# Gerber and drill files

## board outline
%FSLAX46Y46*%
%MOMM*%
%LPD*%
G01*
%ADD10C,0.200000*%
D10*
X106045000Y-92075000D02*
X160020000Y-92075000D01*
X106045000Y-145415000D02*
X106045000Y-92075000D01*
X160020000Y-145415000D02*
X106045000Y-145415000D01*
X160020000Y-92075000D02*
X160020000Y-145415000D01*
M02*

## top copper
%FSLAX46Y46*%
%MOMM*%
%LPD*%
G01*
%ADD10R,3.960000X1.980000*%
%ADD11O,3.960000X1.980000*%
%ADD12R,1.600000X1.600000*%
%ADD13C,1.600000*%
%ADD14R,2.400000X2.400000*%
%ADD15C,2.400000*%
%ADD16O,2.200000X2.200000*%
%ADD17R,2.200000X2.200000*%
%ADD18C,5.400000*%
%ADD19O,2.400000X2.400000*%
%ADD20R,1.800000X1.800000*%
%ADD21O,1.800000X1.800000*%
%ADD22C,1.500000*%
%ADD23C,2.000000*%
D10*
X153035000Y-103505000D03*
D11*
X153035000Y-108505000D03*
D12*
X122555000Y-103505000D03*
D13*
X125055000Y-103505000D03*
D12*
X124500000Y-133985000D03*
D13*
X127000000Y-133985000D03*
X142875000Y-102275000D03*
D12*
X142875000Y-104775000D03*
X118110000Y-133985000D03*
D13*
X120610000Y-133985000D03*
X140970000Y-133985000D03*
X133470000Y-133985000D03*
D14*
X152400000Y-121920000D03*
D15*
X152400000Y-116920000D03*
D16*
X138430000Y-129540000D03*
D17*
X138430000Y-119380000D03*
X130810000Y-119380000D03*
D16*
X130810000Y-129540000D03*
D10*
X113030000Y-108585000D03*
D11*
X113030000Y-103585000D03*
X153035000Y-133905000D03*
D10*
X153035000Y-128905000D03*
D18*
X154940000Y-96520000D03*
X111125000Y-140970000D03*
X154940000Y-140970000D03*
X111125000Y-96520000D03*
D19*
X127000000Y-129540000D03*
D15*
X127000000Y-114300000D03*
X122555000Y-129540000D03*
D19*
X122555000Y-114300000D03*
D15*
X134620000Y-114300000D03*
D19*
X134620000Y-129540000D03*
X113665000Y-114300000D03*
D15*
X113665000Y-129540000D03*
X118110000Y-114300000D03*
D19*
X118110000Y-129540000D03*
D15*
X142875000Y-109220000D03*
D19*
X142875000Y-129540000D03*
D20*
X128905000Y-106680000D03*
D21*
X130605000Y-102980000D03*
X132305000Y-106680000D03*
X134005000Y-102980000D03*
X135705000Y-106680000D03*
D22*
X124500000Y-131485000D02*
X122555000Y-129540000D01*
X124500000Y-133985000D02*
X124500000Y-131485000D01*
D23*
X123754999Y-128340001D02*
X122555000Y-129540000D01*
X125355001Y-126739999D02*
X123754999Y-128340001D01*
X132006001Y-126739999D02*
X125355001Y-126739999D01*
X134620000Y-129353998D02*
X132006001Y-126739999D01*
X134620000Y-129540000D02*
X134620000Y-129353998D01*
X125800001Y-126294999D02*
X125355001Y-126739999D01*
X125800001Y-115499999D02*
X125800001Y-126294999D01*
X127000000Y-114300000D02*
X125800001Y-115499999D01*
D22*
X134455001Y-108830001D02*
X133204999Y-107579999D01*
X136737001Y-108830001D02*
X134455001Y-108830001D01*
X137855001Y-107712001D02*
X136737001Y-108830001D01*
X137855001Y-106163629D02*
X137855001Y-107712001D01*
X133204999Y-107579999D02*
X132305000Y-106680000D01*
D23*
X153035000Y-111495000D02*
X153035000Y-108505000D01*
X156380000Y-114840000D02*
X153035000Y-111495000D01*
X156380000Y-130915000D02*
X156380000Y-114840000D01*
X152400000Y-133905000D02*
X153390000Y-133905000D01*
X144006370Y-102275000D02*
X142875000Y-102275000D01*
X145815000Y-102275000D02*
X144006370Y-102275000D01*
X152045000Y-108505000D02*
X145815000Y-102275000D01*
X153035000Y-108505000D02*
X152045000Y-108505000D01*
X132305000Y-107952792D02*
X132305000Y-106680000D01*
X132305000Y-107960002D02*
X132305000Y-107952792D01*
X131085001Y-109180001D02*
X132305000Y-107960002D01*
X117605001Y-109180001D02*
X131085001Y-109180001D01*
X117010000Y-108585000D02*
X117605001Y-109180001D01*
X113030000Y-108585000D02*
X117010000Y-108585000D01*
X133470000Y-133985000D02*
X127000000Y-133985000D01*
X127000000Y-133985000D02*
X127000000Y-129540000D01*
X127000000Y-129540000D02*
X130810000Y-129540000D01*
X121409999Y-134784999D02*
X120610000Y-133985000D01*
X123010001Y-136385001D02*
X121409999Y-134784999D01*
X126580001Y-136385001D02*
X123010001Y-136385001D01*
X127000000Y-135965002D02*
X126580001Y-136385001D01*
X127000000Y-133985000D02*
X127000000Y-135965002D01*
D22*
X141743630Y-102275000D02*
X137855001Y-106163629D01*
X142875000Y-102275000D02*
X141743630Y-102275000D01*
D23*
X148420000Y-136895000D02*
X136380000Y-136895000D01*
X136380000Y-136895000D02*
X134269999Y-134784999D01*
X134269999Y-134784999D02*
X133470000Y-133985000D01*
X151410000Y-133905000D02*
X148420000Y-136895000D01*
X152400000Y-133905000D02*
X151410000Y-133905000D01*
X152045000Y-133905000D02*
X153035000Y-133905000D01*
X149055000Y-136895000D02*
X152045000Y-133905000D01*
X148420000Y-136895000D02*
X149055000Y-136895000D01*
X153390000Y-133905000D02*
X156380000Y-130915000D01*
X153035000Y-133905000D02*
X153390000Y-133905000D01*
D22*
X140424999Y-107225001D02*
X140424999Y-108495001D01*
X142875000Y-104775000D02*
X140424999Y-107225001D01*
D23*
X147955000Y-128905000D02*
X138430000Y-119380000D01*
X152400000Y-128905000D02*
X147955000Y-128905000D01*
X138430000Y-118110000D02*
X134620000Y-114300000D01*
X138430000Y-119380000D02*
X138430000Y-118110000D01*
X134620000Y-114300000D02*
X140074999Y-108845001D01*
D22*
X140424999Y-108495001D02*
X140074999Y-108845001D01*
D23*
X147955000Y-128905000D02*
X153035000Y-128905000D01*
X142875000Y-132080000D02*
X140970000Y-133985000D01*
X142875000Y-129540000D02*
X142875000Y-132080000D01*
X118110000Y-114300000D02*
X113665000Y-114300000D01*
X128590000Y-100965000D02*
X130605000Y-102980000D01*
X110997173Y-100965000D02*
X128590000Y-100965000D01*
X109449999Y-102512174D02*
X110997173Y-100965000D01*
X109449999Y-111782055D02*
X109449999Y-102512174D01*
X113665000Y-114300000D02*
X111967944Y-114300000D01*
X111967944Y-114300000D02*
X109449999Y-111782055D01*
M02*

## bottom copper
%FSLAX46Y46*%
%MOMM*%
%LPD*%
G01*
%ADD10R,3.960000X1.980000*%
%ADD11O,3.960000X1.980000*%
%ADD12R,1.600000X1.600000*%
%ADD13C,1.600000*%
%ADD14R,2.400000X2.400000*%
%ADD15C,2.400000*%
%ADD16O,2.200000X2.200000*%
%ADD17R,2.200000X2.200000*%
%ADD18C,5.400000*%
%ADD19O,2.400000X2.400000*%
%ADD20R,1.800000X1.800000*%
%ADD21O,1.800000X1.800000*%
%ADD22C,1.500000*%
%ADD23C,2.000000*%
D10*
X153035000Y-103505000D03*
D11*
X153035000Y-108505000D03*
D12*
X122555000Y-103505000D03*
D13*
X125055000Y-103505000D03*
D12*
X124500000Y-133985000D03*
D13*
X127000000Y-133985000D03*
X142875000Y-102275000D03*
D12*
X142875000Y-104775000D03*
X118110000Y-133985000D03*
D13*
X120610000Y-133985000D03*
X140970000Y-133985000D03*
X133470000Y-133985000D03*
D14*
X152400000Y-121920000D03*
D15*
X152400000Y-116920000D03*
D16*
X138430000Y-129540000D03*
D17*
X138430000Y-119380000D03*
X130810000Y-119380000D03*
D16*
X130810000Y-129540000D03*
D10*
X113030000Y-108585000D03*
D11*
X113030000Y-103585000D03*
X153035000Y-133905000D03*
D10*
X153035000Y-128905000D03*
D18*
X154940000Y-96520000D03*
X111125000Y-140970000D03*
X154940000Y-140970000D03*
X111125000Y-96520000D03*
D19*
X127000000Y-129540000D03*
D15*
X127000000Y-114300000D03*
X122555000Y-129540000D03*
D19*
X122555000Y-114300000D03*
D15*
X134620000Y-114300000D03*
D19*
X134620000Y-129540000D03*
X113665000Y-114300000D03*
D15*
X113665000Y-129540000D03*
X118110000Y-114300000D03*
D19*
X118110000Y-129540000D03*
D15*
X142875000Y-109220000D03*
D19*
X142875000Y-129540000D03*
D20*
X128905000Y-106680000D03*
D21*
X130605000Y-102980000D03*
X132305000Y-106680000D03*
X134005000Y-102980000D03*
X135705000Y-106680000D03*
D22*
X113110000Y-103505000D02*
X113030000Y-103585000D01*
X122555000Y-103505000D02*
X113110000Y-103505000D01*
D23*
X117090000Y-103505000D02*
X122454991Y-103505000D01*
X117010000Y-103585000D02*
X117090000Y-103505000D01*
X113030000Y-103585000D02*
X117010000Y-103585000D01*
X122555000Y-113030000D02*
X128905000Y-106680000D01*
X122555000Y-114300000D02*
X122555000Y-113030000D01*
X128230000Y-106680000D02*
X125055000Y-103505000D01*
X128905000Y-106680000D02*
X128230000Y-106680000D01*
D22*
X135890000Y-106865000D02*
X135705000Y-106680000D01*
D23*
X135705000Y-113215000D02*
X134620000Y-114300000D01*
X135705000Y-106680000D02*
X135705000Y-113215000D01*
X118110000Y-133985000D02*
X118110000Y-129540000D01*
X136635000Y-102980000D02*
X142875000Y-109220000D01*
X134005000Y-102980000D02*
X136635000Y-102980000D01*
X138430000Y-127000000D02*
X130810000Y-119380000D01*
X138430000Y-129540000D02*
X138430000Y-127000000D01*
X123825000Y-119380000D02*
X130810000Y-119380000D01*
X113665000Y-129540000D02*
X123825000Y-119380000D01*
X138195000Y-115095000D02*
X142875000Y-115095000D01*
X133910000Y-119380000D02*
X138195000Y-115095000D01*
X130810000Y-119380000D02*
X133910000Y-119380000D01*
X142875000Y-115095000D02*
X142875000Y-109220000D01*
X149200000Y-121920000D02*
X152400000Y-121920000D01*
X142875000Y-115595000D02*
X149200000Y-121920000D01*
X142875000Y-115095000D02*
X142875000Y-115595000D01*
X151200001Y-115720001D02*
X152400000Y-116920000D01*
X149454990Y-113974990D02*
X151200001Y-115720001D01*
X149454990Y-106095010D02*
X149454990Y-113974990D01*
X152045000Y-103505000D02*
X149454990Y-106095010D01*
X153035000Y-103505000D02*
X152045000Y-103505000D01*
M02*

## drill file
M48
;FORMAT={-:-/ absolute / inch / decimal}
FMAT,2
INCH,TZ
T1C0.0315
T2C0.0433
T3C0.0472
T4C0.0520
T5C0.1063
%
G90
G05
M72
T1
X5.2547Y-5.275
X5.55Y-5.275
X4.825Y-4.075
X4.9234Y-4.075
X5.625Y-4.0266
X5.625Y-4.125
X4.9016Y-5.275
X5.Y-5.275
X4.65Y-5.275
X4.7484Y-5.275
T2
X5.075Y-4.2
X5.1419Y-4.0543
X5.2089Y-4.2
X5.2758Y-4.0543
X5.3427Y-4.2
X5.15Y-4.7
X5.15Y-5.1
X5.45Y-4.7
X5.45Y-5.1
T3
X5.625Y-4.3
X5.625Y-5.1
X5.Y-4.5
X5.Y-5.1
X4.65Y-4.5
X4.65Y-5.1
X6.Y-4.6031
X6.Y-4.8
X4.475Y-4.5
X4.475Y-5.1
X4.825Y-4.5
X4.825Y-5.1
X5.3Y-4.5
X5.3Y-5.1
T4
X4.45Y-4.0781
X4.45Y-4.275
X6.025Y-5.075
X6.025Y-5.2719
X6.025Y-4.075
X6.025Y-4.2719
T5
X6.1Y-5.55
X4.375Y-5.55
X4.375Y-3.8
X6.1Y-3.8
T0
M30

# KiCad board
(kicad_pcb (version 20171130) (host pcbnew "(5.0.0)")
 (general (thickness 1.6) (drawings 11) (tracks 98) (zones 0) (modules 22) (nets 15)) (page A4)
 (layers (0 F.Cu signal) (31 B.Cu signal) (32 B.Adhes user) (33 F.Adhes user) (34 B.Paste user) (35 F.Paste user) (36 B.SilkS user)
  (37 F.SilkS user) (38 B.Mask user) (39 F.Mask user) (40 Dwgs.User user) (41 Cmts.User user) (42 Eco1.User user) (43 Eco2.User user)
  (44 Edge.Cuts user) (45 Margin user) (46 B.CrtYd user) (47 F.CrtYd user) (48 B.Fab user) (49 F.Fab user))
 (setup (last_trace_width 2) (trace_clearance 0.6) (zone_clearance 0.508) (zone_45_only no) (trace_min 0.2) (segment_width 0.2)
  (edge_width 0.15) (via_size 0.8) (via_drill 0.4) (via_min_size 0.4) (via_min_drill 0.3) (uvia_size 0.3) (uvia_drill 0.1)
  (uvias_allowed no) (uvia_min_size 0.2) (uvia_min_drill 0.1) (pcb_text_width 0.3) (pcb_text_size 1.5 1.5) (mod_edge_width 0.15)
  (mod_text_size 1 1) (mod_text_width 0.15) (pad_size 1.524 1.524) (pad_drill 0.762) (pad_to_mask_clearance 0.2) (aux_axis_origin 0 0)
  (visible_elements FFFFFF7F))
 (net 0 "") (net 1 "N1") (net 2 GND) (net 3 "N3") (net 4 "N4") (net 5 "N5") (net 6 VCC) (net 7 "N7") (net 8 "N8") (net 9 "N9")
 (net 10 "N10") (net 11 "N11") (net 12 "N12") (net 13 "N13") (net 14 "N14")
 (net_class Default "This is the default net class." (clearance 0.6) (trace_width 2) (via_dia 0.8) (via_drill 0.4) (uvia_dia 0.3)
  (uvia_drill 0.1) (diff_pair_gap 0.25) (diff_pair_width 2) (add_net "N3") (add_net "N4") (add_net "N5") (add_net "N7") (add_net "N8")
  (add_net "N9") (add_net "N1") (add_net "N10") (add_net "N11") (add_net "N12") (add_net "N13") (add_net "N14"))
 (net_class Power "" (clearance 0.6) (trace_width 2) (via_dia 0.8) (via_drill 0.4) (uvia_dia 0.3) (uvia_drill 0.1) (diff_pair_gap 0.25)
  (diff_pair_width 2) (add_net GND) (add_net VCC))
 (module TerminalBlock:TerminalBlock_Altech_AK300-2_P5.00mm (layer F.Cu) (at 153.035 103.505 270)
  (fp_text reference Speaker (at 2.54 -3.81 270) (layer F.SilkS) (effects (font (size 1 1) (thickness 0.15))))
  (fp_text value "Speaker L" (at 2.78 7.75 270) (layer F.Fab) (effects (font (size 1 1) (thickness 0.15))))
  (pad 1 thru_hole rect (at 0 0 270) (size 1.98 3.96) (drill 1.32) (layers *.Cu *.Mask) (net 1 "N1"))
  (pad 2 thru_hole oval (at 5 0 270) (size 1.98 3.96) (drill 1.32) (layers *.Cu *.Mask) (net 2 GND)))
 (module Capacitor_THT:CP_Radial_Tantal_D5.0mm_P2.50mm (layer F.Cu) (at 122.555 103.505)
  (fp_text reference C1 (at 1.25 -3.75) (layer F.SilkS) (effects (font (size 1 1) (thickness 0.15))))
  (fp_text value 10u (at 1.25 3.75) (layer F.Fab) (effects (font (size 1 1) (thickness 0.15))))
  (pad 1 thru_hole rect (at 0 0) (size 1.6 1.6) (drill 0.8) (layers *.Cu *.Mask) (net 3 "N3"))
  (pad 2 thru_hole circle (at 2.5 0) (size 1.6 1.6) (drill 0.8) (layers *.Cu *.Mask) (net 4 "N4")))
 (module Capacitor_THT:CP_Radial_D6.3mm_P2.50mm (layer F.Cu) (at 124.5 133.985)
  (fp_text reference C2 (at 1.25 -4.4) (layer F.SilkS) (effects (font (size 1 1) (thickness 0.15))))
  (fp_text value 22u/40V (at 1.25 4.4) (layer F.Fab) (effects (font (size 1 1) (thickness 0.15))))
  (pad 1 thru_hole rect (at 0 0) (size 1.6 1.6) (drill 0.8) (layers *.Cu *.Mask) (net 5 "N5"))
  (pad 2 thru_hole circle (at 2.5 0) (size 1.6 1.6) (drill 0.8) (layers *.Cu *.Mask) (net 2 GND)))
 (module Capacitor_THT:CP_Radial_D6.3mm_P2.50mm (layer F.Cu) (at 142.875 104.775 90)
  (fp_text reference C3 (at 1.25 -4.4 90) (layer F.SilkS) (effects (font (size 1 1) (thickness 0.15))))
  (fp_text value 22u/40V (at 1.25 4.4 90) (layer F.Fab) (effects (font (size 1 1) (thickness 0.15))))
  (pad 2 thru_hole circle (at 2.5 0 90) (size 1.6 1.6) (drill 0.8) (layers *.Cu *.Mask) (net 2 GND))
  (pad 1 thru_hole rect (at 0 0 90) (size 1.6 1.6) (drill 0.8) (layers *.Cu *.Mask) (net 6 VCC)))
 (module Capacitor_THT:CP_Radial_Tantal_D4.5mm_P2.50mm (layer F.Cu) (at 118.11 133.985)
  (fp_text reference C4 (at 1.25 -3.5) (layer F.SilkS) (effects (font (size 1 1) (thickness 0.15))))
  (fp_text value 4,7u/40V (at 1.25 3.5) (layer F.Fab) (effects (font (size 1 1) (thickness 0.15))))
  (pad 1 thru_hole rect (at 0 0) (size 1.6 1.6) (drill 0.8) (layers *.Cu *.Mask) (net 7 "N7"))
  (pad 2 thru_hole circle (at 2.5 0) (size 1.6 1.6) (drill 0.8) (layers *.Cu *.Mask) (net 2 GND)))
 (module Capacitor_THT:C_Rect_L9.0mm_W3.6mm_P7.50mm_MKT (layer F.Cu) (at 140.97 133.985 180)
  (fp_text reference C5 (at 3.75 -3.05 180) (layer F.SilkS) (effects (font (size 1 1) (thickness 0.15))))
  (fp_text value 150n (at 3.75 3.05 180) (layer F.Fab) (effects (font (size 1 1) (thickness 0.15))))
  (pad 1 thru_hole circle (at 0 0 180) (size 1.6 1.6) (drill 0.8) (layers *.Cu *.Mask) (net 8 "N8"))
  (pad 2 thru_hole circle (at 7.5 0 180) (size 1.6 1.6) (drill 0.8) (layers *.Cu *.Mask) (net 2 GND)))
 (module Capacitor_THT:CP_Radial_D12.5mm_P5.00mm (layer F.Cu) (at 152.4 121.92 90)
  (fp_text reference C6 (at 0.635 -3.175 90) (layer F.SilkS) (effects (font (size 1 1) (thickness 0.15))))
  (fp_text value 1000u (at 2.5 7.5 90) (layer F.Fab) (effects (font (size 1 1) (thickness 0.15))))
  (pad 1 thru_hole rect (at 0 0 90) (size 2.4 2.4) (drill 1.2) (layers *.Cu *.Mask) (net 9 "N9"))
  (pad 2 thru_hole circle (at 5 0 90) (size 2.4 2.4) (drill 1.2) (layers *.Cu *.Mask) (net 1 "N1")))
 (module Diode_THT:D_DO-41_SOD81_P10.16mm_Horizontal (layer F.Cu) (at 138.43 119.38 270)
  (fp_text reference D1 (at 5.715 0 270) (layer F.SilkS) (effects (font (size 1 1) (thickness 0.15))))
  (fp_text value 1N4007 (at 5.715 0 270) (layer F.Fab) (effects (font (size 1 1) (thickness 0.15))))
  (pad 2 thru_hole oval (at 10.16 0 270) (size 2.2 2.2) (drill 1.1) (layers *.Cu *.Mask) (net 9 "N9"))
  (pad 1 thru_hole rect (at 0 0 270) (size 2.2 2.2) (drill 1.1) (layers *.Cu *.Mask) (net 6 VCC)))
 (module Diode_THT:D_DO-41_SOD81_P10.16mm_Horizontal (layer F.Cu) (at 130.81 119.38 270)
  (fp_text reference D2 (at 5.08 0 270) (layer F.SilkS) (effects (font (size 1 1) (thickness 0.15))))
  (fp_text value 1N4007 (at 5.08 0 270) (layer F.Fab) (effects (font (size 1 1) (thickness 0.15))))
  (pad 1 thru_hole rect (at 0 0 270) (size 2.2 2.2) (drill 1.1) (layers *.Cu *.Mask) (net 9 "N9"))
  (pad 2 thru_hole oval (at 10.16 0 270) (size 2.2 2.2) (drill 1.1) (layers *.Cu *.Mask) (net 2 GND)))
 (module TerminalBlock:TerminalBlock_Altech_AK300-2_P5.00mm (layer F.Cu) (at 113.03 108.585 90)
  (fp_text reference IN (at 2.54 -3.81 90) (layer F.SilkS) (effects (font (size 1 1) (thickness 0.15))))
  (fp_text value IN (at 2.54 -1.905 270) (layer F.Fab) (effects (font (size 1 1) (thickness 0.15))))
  (pad 1 thru_hole rect (at 0 0 90) (size 1.98 3.96) (drill 1.32) (layers *.Cu *.Mask) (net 2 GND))
  (pad 2 thru_hole oval (at 5 0 90) (size 1.98 3.96) (drill 1.32) (layers *.Cu *.Mask) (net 3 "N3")))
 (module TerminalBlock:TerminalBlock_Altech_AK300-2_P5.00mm (layer F.Cu) (at 153.035 128.905 270)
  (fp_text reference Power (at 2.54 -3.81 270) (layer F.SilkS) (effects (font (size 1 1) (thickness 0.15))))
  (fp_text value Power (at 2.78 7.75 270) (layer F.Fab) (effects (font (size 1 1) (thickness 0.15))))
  (pad 2 thru_hole oval (at 5 0 270) (size 1.98 3.96) (drill 1.32) (layers *.Cu *.Mask) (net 2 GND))
  (pad 1 thru_hole rect (at 0 0 270) (size 1.98 3.96) (drill 1.32) (layers *.Cu *.Mask) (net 6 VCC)))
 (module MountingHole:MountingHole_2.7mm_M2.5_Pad (layer F.Cu) (at 154.94 96.52)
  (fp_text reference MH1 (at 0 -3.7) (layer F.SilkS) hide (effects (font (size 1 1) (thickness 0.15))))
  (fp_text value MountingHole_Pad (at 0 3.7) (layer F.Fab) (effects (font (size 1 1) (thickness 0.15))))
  (pad 1 thru_hole circle (at 0 0) (size 5.4 5.4) (drill 2.7) (layers *.Cu *.Mask) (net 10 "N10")))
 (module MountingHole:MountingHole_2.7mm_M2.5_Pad (layer F.Cu) (at 111.125 140.97)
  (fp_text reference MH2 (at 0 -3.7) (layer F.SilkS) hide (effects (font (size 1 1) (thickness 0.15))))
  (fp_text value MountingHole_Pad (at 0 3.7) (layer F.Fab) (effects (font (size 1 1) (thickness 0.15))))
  (pad 1 thru_hole circle (at 0 0) (size 5.4 5.4) (drill 2.7) (layers *.Cu *.Mask) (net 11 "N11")))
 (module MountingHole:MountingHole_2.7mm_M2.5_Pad (layer F.Cu) (at 154.94 140.97)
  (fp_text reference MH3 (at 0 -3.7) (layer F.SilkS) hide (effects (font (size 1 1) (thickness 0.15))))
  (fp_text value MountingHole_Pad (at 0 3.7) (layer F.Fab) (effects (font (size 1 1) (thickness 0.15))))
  (pad 1 thru_hole circle (at 0 0) (size 5.4 5.4) (drill 2.7) (layers *.Cu *.Mask) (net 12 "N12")))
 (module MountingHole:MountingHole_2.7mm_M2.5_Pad (layer F.Cu) (at 111.125 96.52)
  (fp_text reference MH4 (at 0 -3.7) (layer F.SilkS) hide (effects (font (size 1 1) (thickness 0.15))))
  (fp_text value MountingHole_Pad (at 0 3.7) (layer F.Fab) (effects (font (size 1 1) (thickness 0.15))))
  (pad 1 thru_hole circle (at 0 0) (size 5.4 5.4) (drill 2.7) (layers *.Cu *.Mask) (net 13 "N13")))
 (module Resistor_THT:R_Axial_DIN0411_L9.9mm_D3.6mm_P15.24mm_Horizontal (layer F.Cu) (at 127 114.3 270)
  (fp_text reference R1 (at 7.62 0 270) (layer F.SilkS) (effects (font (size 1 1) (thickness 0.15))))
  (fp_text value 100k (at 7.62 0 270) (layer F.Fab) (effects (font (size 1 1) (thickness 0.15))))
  (pad 2 thru_hole oval (at 15.24 0 270) (size 2.4 2.4) (drill 1.2) (layers *.Cu *.Mask) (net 2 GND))
  (pad 1 thru_hole circle (at 0 0 270) (size 2.4 2.4) (drill 1.2) (layers *.Cu *.Mask) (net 5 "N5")))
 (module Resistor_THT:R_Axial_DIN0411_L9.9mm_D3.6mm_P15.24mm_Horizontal (layer F.Cu) (at 122.555 129.54 90)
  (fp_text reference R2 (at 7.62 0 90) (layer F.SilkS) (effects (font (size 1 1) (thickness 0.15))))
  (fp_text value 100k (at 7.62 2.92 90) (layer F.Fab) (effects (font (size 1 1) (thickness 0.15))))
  (pad 1 thru_hole circle (at 0 0 90) (size 2.4 2.4) (drill 1.2) (layers *.Cu *.Mask) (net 5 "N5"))
  (pad 2 thru_hole oval (at 15.24 0 90) (size 2.4 2.4) (drill 1.2) (layers *.Cu *.Mask) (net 4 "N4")))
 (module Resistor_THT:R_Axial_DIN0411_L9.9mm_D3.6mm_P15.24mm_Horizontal (layer F.Cu) (at 134.62 114.3 270)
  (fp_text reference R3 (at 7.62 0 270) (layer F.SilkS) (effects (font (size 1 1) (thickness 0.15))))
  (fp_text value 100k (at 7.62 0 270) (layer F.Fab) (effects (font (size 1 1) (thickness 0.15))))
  (pad 1 thru_hole circle (at 0 0 270) (size 2.4 2.4) (drill 1.2) (layers *.Cu *.Mask) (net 6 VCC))
  (pad 2 thru_hole oval (at 15.24 0 270) (size 2.4 2.4) (drill 1.2) (layers *.Cu *.Mask) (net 5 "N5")))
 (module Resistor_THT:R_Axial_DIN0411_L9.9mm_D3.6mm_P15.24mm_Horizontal (layer F.Cu) (at 113.665 129.54 90)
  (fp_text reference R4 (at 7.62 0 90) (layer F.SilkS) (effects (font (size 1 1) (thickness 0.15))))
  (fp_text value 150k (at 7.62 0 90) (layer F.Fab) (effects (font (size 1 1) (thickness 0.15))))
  (pad 2 thru_hole oval (at 15.24 0 90) (size 2.4 2.4) (drill 1.2) (layers *.Cu *.Mask) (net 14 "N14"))
  (pad 1 thru_hole circle (at 0 0 90) (size 2.4 2.4) (drill 1.2) (layers *.Cu *.Mask) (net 9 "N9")))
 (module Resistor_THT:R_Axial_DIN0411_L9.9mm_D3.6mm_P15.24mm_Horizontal (layer F.Cu) (at 118.11 114.3 270)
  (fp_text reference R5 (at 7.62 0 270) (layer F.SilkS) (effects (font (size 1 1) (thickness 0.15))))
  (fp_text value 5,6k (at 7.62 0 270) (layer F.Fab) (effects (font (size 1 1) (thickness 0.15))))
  (pad 1 thru_hole circle (at 0 0 270) (size 2.4 2.4) (drill 1.2) (layers *.Cu *.Mask) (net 14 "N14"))
  (pad 2 thru_hole oval (at 15.24 0 270) (size 2.4 2.4) (drill 1.2) (layers *.Cu *.Mask) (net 7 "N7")))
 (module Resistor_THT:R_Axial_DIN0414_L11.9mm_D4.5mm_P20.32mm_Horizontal (layer F.Cu) (at 142.875 109.22 270)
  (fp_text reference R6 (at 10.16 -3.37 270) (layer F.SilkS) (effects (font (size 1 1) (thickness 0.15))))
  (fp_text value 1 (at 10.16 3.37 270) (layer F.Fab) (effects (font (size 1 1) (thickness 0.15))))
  (pad 1 thru_hole circle (at 0 0 270) (size 2.4 2.4) (drill 1.2) (layers *.Cu *.Mask) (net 9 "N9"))
  (pad 2 thru_hole oval (at 20.32 0 270) (size 2.4 2.4) (drill 1.2) (layers *.Cu *.Mask) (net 8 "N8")))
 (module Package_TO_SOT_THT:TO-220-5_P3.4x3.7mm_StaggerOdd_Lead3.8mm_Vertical (layer F.Cu) (at 128.905 106.68)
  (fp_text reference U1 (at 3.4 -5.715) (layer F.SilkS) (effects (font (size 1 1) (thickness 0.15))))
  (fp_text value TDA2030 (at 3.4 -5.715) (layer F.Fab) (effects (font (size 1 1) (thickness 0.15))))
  (pad 1 thru_hole rect (at 0 0) (size 1.8 1.8) (drill 1.1) (layers *.Cu *.Mask) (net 4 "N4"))
  (pad 2 thru_hole oval (at 1.7 -3.7) (size 1.8 1.8) (drill 1.1) (layers *.Cu *.Mask) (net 14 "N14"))
  (pad 3 thru_hole oval (at 3.4 0) (size 1.8 1.8) (drill 1.1) (layers *.Cu *.Mask) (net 2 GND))
  (pad 4 thru_hole oval (at 5.1 -3.7) (size 1.8 1.8) (drill 1.1) (layers *.Cu *.Mask) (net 9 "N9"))
  (pad 5 thru_hole oval (at 6.8 0) (size 1.8 1.8) (drill 1.1) (layers *.Cu *.Mask) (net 6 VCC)))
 (gr_line (start 106.045 92.075) (end 160.02 92.075) (layer Edge.Cuts) (width 0.2))
 (gr_line (start 106.045 145.415) (end 106.045 92.075) (layer Edge.Cuts) (width 0.2))
 (gr_line (start 160.02 145.415) (end 106.045 145.415) (layer Edge.Cuts) (width 0.2))
 (gr_line (start 160.02 92.075) (end 160.02 145.415) (layer Edge.Cuts) (width 0.2))
 (segment (start 113.11 103.505) (end 113.03 103.585) (width 1.5) (layer B.Cu) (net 3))
 (segment (start 122.555 103.505) (end 113.11 103.505) (width 1.5) (layer B.Cu) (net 3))
 (segment (start 117.09 103.505) (end 122.454991 103.505) (width 2) (layer B.Cu) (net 3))
 (segment (start 117.01 103.585) (end 117.09 103.505) (width 2) (layer B.Cu) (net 3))
 (segment (start 113.03 103.585) (end 117.01 103.585) (width 2) (layer B.Cu) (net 3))
 (segment (start 122.555 113.03) (end 128.905 106.68) (width 2) (layer B.Cu) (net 4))
 (segment (start 122.555 114.3) (end 122.555 113.03) (width 2) (layer B.Cu) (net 4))
 (segment (start 128.23 106.68) (end 125.055 103.505) (width 2) (layer B.Cu) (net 4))
 (segment (start 128.905 106.68) (end 128.23 106.68) (width 2) (layer B.Cu) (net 4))
 (segment (start 124.5 131.485) (end 122.555 129.54) (width 1.5) (layer F.Cu) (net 5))
 (segment (start 124.5 133.985) (end 124.5 131.485) (width 1.5) (layer F.Cu) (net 5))
 (segment (start 123.754999 128.340001) (end 122.555 129.54) (width 2) (layer F.Cu) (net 5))
 (segment (start 125.355001 126.739999) (end 123.754999 128.340001) (width 2) (layer F.Cu) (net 5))
 (segment (start 132.006001 126.739999) (end 125.355001 126.739999) (width 2) (layer F.Cu) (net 5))
 (segment (start 134.62 129.353998) (end 132.006001 126.739999) (width 2) (layer F.Cu) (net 5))
 (segment (start 134.62 129.54) (end 134.62 129.353998) (width 2) (layer F.Cu) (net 5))
 (segment (start 125.800001 126.294999) (end 125.355001 126.739999) (width 2) (layer F.Cu) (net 5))
 (segment (start 125.800001 115.499999) (end 125.800001 126.294999) (width 2) (layer F.Cu) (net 5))
 (segment (start 127 114.3) (end 125.800001 115.499999) (width 2) (layer F.Cu) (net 5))
 (segment (start 134.455001 108.830001) (end 133.204999 107.579999) (width 1.5) (layer F.Cu) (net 2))
 (segment (start 136.737001 108.830001) (end 134.455001 108.830001) (width 1.5) (layer F.Cu) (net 2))
 (segment (start 137.855001 107.712001) (end 136.737001 108.830001) (width 1.5) (layer F.Cu) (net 2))
 (segment (start 137.855001 106.163629) (end 137.855001 107.712001) (width 1.5) (layer F.Cu) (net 2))
 (segment (start 133.204999 107.579999) (end 132.305 106.68) (width 1.5) (layer F.Cu) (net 2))
 (segment (start 153.035 111.495) (end 153.035 108.505) (width 2) (layer F.Cu) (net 2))
 (segment (start 156.38 114.84) (end 153.035 111.495) (width 2) (layer F.Cu) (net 2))
 (segment (start 156.38 130.915) (end 156.38 114.84) (width 2) (layer F.Cu) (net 2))
 (segment (start 152.4 133.905) (end 153.39 133.905) (width 2) (layer F.Cu) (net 2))
 (segment (start 144.00637 102.275) (end 142.875 102.275) (width 2) (layer F.Cu) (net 2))
 (segment (start 145.815 102.275) (end 144.00637 102.275) (width 2) (layer F.Cu) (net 2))
 (segment (start 152.045 108.505) (end 145.815 102.275) (width 2) (layer F.Cu) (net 2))
 (segment (start 153.035 108.505) (end 152.045 108.505) (width 2) (layer F.Cu) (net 2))
 (segment (start 132.305 107.952792) (end 132.305 106.68) (width 2) (layer F.Cu) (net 2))
 (segment (start 132.305 107.960002) (end 132.305 107.952792) (width 2) (layer F.Cu) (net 2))
 (segment (start 131.085001 109.180001) (end 132.305 107.960002) (width 2) (layer F.Cu) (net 2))
 (segment (start 117.605001 109.180001) (end 131.085001 109.180001) (width 2) (layer F.Cu) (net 2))
 (segment (start 117.01 108.585) (end 117.605001 109.180001) (width 2) (layer F.Cu) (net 2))
 (segment (start 113.03 108.585) (end 117.01 108.585) (width 2) (layer F.Cu) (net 2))
 (segment (start 133.47 133.985) (end 127 133.985) (width 2) (layer F.Cu) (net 2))
 (segment (start 127 133.985) (end 127 129.54) (width 2) (layer F.Cu) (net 2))
 (segment (start 127 129.54) (end 130.81 129.54) (width 2) (layer F.Cu) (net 2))
 (segment (start 121.409999 134.784999) (end 120.61 133.985) (width 2) (layer F.Cu) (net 2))
 (segment (start 123.010001 136.385001) (end 121.409999 134.784999) (width 2) (layer F.Cu) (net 2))
 (segment (start 126.580001 136.385001) (end 123.010001 136.385001) (width 2) (layer F.Cu) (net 2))
 (segment (start 127 135.965002) (end 126.580001 136.385001) (width 2) (layer F.Cu) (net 2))
 (segment (start 127 133.985) (end 127 135.965002) (width 2) (layer F.Cu) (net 2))
 (segment (start 141.74363 102.275) (end 137.855001 106.163629) (width 1.5) (layer F.Cu) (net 2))
 (segment (start 142.875 102.275) (end 141.74363 102.275) (width 1.5) (layer F.Cu) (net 2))
 (segment (start 148.42 136.895) (end 136.38 136.895) (width 2) (layer F.Cu) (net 2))
 (segment (start 136.38 136.895) (end 134.269999 134.784999) (width 2) (layer F.Cu) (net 2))
 (segment (start 134.269999 134.784999) (end 133.47 133.985) (width 2) (layer F.Cu) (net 2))
 (segment (start 151.41 133.905) (end 148.42 136.895) (width 2) (layer F.Cu) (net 2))
 (segment (start 152.4 133.905) (end 151.41 133.905) (width 2) (layer F.Cu) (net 2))
 (segment (start 152.045 133.905) (end 153.035 133.905) (width 2) (layer F.Cu) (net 2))
 (segment (start 149.055 136.895) (end 152.045 133.905) (width 2) (layer F.Cu) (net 2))
 (segment (start 148.42 136.895) (end 149.055 136.895) (width 2) (layer F.Cu) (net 2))
 (segment (start 153.39 133.905) (end 156.38 130.915) (width 2) (layer F.Cu) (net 2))
 (segment (start 153.035 133.905) (end 153.39 133.905) (width 2) (layer F.Cu) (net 2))
 (segment (start 135.89 106.865) (end 135.705 106.68) (width 1.5) (layer B.Cu) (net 6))
 (segment (start 140.424999 107.225001) (end 140.424999 108.495001) (width 1.5) (layer F.Cu) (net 6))
 (segment (start 142.875 104.775) (end 140.424999 107.225001) (width 1.5) (layer F.Cu) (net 6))
 (segment (start 147.955 128.905) (end 138.43 119.38) (width 2) (layer F.Cu) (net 6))
 (segment (start 152.4 128.905) (end 147.955 128.905) (width 2) (layer F.Cu) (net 6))
 (segment (start 138.43 118.11) (end 134.62 114.3) (width 2) (layer F.Cu) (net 6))
 (segment (start 138.43 119.38) (end 138.43 118.11) (width 2) (layer F.Cu) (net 6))
 (segment (start 134.62 114.3) (end 140.074999 108.845001) (width 2) (layer F.Cu) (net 6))
 (segment (start 140.424999 108.495001) (end 140.074999 108.845001) (width 1.5) (layer F.Cu) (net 6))
 (segment (start 135.705 113.215) (end 134.62 114.3) (width 2) (layer B.Cu) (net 6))
 (segment (start 135.705 106.68) (end 135.705 113.215) (width 2) (layer B.Cu) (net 6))
 (segment (start 147.955 128.905) (end 153.035 128.905) (width 2) (layer F.Cu) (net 6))
 (segment (start 118.11 133.985) (end 118.11 129.54) (width 2) (layer B.Cu) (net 7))
 (segment (start 142.875 132.08) (end 140.97 133.985) (width 2) (layer F.Cu) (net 8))
 (segment (start 142.875 129.54) (end 142.875 132.08) (width 2) (layer F.Cu) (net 8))
 (segment (start 136.635 102.98) (end 142.875 109.22) (width 2) (layer B.Cu) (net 9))
 (segment (start 134.005 102.98) (end 136.635 102.98) (width 2) (layer B.Cu) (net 9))
 (segment (start 138.43 127) (end 130.81 119.38) (width 2) (layer B.Cu) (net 9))
 (segment (start 138.43 129.54) (end 138.43 127) (width 2) (layer B.Cu) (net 9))
 (segment (start 123.825 119.38) (end 130.81 119.38) (width 2) (layer B.Cu) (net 9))
 (segment (start 113.665 129.54) (end 123.825 119.38) (width 2) (layer B.Cu) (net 9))
 (segment (start 138.195 115.095) (end 142.875 115.095) (width 2) (layer B.Cu) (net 9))
 (segment (start 133.91 119.38) (end 138.195 115.095) (width 2) (layer B.Cu) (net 9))
 (segment (start 130.81 119.38) (end 133.91 119.38) (width 2) (layer B.Cu) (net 9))
 (segment (start 142.875 115.095) (end 142.875 109.22) (width 2) (layer B.Cu) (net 9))
 (segment (start 149.2 121.92) (end 152.4 121.92) (width 2) (layer B.Cu) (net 9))
 (segment (start 142.875 115.595) (end 149.2 121.92) (width 2) (layer B.Cu) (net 9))
 (segment (start 142.875 115.095) (end 142.875 115.595) (width 2) (layer B.Cu) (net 9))
 (segment (start 151.200001 115.720001) (end 152.4 116.92) (width 2) (layer B.Cu) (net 1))
 (segment (start 149.45499 113.97499) (end 151.200001 115.720001) (width 2) (layer B.Cu) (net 1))
 (segment (start 149.45499 106.09501) (end 149.45499 113.97499) (width 2) (layer B.Cu) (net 1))
 (segment (start 152.045 103.505) (end 149.45499 106.09501) (width 2) (layer B.Cu) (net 1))
 (segment (start 153.035 103.505) (end 152.045 103.505) (width 2) (layer B.Cu) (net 1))
 (segment (start 118.11 114.3) (end 113.665 114.3) (width 2) (layer F.Cu) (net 14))
 (segment (start 128.59 100.965) (end 130.605 102.98) (width 2) (layer F.Cu) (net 14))
 (segment (start 110.997173 100.965) (end 128.59 100.965) (width 2) (layer F.Cu) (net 14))
 (segment (start 109.449999 102.512174) (end 110.997173 100.965) (width 2) (layer F.Cu) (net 14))
 (segment (start 109.449999 111.782055) (end 109.449999 102.512174) (width 2) (layer F.Cu) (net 14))
 (segment (start 113.665 114.3) (end 111.967944 114.3) (width 2) (layer F.Cu) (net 14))
 (segment (start 111.967944 114.3) (end 109.449999 111.782055) (width 2) (layer F.Cu) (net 14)))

